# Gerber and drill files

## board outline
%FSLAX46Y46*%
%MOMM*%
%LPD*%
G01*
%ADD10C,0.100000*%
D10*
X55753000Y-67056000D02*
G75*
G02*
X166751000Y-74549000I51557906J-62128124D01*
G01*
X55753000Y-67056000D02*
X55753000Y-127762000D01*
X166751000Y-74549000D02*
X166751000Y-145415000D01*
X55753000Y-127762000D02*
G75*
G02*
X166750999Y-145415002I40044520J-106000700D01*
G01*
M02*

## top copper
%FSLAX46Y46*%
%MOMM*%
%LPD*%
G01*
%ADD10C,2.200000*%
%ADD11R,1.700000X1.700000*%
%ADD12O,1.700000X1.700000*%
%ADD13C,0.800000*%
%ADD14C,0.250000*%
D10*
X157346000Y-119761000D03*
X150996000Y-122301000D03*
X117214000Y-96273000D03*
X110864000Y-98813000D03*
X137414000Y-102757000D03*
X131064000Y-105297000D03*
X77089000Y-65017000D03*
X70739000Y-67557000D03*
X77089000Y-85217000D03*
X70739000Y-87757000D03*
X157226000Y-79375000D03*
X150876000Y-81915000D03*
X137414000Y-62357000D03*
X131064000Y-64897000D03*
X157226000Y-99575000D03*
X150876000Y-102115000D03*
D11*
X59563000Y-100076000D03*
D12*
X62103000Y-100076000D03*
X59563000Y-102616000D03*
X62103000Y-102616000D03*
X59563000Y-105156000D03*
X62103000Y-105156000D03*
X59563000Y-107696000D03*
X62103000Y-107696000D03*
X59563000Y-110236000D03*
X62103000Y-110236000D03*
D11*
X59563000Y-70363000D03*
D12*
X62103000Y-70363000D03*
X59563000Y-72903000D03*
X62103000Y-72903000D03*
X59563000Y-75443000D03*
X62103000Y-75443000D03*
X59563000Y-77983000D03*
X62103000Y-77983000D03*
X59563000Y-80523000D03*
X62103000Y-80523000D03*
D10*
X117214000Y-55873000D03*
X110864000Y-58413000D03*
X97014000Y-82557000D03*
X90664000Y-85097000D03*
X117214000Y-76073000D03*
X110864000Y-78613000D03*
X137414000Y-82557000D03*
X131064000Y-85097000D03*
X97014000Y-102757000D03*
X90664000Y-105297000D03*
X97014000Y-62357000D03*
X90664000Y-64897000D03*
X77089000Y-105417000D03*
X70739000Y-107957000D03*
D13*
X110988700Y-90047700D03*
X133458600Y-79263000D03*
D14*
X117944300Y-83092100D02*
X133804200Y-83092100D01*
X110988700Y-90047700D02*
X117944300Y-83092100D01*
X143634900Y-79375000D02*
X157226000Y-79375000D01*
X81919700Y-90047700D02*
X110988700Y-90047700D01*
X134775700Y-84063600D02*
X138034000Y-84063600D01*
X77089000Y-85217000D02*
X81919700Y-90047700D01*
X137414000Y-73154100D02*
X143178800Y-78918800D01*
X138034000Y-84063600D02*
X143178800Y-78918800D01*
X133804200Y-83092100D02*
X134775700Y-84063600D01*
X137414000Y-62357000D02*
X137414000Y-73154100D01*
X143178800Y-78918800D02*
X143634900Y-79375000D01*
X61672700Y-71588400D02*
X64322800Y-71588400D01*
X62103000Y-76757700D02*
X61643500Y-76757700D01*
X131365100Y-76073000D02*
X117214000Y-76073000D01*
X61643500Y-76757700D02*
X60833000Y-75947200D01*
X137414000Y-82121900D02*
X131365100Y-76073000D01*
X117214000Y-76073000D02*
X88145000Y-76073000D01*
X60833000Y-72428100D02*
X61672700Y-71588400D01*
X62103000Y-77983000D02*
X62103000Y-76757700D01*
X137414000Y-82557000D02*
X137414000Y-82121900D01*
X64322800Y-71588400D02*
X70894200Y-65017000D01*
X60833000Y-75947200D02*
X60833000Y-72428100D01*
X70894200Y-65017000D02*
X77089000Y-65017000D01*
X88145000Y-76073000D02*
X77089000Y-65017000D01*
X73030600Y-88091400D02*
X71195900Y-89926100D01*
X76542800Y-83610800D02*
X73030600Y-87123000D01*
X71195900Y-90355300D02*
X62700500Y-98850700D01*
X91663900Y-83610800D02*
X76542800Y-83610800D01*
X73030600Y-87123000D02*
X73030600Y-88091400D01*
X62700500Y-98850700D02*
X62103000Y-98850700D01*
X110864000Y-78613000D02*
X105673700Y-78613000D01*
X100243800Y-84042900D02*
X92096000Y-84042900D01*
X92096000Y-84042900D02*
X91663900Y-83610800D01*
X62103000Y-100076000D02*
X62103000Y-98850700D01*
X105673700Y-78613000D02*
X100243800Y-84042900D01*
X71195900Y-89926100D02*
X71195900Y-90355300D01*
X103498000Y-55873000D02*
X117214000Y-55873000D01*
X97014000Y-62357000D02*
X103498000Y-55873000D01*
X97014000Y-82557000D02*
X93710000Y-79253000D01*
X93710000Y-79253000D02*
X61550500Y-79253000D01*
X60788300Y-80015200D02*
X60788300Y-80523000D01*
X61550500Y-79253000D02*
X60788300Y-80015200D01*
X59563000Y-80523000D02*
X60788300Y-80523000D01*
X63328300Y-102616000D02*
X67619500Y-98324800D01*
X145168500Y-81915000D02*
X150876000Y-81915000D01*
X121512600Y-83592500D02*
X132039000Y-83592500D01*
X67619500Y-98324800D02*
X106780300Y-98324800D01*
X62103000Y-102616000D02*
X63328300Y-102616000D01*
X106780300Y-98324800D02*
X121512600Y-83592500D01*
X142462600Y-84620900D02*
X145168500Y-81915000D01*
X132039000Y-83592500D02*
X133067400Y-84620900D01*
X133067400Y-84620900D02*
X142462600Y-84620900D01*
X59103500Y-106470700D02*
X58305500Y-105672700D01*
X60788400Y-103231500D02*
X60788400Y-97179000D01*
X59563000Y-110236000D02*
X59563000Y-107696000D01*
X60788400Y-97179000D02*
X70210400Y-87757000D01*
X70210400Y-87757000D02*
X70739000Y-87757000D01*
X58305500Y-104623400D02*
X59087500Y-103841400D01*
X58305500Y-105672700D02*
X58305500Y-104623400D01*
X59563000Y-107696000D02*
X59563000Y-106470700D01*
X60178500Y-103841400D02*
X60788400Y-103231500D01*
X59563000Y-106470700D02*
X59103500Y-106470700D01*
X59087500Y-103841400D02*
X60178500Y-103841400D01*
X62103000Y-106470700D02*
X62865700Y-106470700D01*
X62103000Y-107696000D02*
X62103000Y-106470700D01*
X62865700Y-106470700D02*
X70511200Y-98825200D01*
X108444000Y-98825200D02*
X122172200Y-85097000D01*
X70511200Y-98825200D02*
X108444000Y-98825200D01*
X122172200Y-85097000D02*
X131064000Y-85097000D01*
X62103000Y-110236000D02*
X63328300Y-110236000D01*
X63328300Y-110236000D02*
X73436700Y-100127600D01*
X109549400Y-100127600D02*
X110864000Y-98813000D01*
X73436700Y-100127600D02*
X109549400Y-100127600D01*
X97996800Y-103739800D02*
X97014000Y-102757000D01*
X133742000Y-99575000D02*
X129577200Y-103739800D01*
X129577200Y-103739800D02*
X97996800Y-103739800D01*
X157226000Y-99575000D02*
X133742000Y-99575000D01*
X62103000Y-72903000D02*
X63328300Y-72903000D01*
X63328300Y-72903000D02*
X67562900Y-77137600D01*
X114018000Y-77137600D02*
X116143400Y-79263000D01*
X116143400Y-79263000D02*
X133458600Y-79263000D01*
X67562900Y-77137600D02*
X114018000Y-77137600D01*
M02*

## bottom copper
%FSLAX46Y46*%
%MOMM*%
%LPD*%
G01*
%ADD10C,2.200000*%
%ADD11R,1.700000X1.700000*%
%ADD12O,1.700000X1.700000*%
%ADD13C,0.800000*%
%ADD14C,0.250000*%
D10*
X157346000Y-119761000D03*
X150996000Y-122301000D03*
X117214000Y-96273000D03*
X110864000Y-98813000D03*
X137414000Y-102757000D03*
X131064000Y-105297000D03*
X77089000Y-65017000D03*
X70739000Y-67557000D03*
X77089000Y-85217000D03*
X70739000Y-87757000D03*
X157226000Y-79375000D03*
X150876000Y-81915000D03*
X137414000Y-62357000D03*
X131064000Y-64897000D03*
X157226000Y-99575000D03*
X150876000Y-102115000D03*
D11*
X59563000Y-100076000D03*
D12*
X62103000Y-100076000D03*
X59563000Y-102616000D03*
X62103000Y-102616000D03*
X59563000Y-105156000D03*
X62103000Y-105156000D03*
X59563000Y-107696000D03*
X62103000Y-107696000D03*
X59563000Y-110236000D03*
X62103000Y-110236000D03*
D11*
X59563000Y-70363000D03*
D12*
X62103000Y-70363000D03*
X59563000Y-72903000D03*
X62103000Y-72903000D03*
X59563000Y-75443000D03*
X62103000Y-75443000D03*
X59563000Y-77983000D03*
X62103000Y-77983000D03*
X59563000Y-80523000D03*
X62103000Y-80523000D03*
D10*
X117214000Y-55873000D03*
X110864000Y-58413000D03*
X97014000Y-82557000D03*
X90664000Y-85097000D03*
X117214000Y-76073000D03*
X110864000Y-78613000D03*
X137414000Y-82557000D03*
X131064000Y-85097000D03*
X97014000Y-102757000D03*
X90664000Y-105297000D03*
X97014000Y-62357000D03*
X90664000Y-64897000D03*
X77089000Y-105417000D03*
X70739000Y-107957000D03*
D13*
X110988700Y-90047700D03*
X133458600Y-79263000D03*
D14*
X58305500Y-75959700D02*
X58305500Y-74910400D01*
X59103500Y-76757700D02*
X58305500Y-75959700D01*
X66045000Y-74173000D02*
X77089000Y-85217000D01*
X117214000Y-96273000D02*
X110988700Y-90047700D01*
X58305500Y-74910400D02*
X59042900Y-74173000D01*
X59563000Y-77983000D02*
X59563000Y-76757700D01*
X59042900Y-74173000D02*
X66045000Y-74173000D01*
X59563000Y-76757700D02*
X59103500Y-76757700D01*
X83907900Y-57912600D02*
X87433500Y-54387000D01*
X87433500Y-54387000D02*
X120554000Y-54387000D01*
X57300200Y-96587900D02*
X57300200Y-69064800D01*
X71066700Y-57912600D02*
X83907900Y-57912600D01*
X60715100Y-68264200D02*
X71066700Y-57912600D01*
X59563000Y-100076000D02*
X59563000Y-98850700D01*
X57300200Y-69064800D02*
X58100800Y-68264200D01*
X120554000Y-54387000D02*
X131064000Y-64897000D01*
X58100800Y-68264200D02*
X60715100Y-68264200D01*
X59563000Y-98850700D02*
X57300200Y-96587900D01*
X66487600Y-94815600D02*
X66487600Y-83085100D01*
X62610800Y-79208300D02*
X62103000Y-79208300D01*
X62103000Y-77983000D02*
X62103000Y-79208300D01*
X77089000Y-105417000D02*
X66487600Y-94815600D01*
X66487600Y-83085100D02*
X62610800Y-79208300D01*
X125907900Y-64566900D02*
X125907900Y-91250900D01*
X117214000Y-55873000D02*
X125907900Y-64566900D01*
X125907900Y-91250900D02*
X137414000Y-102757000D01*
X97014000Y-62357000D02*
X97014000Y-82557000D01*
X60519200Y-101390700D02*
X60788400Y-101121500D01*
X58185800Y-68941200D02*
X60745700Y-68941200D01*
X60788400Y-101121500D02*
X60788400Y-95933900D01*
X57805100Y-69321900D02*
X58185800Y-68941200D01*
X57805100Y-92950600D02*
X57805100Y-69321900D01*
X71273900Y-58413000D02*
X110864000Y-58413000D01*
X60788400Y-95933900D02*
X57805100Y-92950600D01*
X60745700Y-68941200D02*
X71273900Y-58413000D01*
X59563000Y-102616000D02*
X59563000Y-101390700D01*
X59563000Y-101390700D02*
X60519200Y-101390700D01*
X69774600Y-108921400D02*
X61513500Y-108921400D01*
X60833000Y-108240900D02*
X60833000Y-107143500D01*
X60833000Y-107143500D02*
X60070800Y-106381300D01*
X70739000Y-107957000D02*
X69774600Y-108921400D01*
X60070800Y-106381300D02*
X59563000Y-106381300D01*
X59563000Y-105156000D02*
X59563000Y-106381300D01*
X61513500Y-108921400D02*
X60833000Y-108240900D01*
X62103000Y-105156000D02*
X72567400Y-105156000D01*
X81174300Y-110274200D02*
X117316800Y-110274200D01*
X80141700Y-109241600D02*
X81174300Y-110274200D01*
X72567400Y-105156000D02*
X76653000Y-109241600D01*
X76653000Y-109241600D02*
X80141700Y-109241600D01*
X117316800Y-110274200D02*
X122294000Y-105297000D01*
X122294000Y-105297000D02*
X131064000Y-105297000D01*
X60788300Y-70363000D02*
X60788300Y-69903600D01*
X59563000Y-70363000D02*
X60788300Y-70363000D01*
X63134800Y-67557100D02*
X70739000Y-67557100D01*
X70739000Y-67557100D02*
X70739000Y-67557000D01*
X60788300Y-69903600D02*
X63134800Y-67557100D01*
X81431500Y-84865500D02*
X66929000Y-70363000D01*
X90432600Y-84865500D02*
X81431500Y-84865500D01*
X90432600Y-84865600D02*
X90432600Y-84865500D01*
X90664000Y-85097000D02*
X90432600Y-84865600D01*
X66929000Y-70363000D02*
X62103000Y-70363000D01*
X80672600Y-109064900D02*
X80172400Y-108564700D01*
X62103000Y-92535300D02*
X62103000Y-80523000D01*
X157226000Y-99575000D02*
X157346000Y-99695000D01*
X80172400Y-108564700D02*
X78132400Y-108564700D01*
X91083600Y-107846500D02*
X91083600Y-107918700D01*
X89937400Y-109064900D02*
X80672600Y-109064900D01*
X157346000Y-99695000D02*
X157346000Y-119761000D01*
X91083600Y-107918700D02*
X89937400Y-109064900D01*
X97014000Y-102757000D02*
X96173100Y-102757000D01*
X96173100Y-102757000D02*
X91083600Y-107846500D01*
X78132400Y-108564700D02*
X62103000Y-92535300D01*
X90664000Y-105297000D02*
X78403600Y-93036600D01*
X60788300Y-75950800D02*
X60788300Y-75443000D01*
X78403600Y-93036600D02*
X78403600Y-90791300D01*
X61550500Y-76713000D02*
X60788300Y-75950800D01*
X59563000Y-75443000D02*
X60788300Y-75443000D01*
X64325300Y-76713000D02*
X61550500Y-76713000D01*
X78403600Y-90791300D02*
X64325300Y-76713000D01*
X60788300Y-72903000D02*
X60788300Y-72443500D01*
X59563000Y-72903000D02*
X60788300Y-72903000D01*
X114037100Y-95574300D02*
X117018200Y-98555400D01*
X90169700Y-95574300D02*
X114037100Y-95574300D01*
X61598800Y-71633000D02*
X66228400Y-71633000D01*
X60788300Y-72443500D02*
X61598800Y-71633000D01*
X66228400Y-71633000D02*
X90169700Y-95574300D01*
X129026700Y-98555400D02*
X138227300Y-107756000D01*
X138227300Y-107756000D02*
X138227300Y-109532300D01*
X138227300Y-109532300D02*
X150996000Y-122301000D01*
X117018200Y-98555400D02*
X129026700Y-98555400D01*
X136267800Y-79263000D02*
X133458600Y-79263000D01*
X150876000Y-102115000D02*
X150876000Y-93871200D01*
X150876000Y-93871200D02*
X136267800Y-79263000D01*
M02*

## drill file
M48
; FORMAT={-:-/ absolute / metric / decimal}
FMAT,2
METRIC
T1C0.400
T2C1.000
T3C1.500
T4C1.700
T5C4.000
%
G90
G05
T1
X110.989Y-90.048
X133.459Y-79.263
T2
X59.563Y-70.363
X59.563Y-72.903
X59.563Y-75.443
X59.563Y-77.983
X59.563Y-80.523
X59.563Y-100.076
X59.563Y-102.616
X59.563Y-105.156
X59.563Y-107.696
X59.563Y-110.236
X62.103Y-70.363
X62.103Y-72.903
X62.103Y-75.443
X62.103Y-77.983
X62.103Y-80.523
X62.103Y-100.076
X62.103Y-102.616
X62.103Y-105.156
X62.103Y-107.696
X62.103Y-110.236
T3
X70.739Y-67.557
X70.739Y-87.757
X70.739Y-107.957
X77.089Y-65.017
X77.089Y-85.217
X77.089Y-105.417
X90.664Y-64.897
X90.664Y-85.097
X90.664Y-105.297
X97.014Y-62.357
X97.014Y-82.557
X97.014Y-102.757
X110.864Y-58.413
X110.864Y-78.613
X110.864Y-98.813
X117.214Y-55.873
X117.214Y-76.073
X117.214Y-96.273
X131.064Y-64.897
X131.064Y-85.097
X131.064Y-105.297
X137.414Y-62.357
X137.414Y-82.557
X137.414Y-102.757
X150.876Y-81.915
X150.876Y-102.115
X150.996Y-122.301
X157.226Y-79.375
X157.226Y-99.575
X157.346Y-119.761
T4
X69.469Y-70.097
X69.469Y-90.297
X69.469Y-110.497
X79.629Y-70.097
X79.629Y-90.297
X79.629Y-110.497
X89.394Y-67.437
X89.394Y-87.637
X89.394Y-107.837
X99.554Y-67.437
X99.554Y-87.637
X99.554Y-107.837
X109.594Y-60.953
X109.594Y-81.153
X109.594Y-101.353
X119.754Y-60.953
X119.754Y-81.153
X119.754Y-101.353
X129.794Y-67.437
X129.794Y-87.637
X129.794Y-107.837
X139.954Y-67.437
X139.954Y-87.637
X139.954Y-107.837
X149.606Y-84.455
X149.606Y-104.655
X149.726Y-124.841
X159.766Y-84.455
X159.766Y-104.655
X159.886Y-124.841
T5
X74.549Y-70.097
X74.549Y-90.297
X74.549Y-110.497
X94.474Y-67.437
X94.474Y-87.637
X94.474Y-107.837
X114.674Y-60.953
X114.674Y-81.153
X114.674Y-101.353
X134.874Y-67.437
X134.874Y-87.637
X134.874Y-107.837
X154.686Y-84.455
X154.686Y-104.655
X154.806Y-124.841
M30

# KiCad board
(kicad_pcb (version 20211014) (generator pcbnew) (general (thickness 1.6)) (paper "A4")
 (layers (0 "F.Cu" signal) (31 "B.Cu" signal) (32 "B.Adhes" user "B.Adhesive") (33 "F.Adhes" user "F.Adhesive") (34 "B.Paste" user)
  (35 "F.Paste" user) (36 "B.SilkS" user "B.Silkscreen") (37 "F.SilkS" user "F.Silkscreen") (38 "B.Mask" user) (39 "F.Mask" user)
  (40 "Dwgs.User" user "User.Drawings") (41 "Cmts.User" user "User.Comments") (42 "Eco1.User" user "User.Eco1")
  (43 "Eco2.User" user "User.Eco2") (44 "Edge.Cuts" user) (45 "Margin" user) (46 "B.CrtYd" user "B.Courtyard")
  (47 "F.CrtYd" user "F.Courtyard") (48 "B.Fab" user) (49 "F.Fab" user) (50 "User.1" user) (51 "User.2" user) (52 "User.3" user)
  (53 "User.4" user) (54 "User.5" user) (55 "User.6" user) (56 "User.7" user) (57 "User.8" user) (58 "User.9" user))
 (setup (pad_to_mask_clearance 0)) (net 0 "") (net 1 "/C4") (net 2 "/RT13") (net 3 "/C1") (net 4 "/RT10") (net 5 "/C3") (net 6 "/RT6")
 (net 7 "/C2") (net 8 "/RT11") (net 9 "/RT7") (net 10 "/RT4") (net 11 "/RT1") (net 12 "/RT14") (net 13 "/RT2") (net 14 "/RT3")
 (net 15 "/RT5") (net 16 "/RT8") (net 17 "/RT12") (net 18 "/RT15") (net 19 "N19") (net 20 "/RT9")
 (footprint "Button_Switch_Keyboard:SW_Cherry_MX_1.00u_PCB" (layer "F.Cu") (at 157.346 119.761)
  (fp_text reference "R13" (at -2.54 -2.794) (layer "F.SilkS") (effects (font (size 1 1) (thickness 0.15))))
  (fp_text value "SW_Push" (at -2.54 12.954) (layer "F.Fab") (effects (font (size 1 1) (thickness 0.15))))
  (pad "" np_thru_hole circle (at 2.54 5.08) (size 1.7 1.7) (drill 1.7) (layers *.Cu *.Mask))
  (pad "" np_thru_hole circle (at -2.54 5.08) (size 4 4) (drill 4) (layers *.Cu *.Mask))
  (pad "" np_thru_hole circle (at -7.62 5.08) (size 1.7 1.7) (drill 1.7) (layers *.Cu *.Mask))
  (pad "1" thru_hole circle (at 0 0) (size 2.2 2.2) (drill 1.5) (layers *.Cu *.Mask) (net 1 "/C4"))
  (pad "2" thru_hole circle (at -6.35 2.54) (size 2.2 2.2) (drill 1.5) (layers *.Cu *.Mask) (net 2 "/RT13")))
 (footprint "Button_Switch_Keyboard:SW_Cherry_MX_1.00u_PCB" (layer "F.Cu") (at 117.214 96.273)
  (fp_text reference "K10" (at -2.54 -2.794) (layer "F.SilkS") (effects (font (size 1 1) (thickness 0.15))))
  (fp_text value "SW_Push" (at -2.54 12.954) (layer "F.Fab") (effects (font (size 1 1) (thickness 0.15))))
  (pad "" np_thru_hole circle (at 2.54 5.08) (size 1.7 1.7) (drill 1.7) (layers *.Cu *.Mask))
  (pad "" np_thru_hole circle (at -7.62 5.08) (size 1.7 1.7) (drill 1.7) (layers *.Cu *.Mask))
  (pad "" np_thru_hole circle (at -2.54 5.08) (size 4 4) (drill 4) (layers *.Cu *.Mask))
  (pad "1" thru_hole circle (at 0 0) (size 2.2 2.2) (drill 1.5) (layers *.Cu *.Mask) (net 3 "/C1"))
  (pad "2" thru_hole circle (at -6.35 2.54) (size 2.2 2.2) (drill 1.5) (layers *.Cu *.Mask) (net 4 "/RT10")))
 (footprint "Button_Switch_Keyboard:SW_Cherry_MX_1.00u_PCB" (layer "F.Cu") (at 137.414 102.757)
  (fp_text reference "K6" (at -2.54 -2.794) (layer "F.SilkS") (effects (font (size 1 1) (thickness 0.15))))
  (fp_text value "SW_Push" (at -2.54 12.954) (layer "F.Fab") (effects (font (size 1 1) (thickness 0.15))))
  (pad "" np_thru_hole circle (at -7.62 5.08) (size 1.7 1.7) (drill 1.7) (layers *.Cu *.Mask))
  (pad "" np_thru_hole circle (at 2.54 5.08) (size 1.7 1.7) (drill 1.7) (layers *.Cu *.Mask))
  (pad "" np_thru_hole circle (at -2.54 5.08) (size 4 4) (drill 4) (layers *.Cu *.Mask))
  (pad "1" thru_hole circle (at 0 0) (size 2.2 2.2) (drill 1.5) (layers *.Cu *.Mask) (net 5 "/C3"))
  (pad "2" thru_hole circle (at -6.35 2.54) (size 2.2 2.2) (drill 1.5) (layers *.Cu *.Mask) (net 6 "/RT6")))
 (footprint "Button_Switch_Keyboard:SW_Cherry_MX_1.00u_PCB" (layer "F.Cu") (at 77.089 65.017)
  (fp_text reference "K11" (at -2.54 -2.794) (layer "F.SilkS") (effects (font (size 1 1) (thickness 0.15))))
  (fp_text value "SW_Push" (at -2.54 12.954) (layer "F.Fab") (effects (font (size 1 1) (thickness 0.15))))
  (pad "" np_thru_hole circle (at 2.54 5.08) (size 1.7 1.7) (drill 1.7) (layers *.Cu *.Mask))
  (pad "" np_thru_hole circle (at -7.62 5.08) (size 1.7 1.7) (drill 1.7) (layers *.Cu *.Mask))
  (pad "" np_thru_hole circle (at -2.54 5.08) (size 4 4) (drill 4) (layers *.Cu *.Mask))
  (pad "1" thru_hole circle (at 0 0) (size 2.2 2.2) (drill 1.5) (layers *.Cu *.Mask) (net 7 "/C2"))
  (pad "2" thru_hole circle (at -6.35 2.54) (size 2.2 2.2) (drill 1.5) (layers *.Cu *.Mask) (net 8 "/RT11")))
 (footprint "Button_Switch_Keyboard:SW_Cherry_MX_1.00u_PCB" (layer "F.Cu") (at 77.089 85.217)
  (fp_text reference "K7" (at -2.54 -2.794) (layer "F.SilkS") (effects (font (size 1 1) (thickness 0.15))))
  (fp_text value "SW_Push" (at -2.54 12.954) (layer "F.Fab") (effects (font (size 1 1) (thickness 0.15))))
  (pad "" np_thru_hole circle (at -7.62 5.08) (size 1.7 1.7) (drill 1.7) (layers *.Cu *.Mask))
  (pad "" np_thru_hole circle (at -2.54 5.08) (size 4 4) (drill 4) (layers *.Cu *.Mask))
  (pad "" np_thru_hole circle (at 2.54 5.08) (size 1.7 1.7) (drill 1.7) (layers *.Cu *.Mask))
  (pad "1" thru_hole circle (at 0 0) (size 2.2 2.2) (drill 1.5) (layers *.Cu *.Mask) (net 3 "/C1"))
  (pad "2" thru_hole circle (at -6.35 2.54) (size 2.2 2.2) (drill 1.5) (layers *.Cu *.Mask) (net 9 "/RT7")))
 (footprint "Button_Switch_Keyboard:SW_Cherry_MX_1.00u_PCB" (layer "F.Cu") (at 157.226 79.375)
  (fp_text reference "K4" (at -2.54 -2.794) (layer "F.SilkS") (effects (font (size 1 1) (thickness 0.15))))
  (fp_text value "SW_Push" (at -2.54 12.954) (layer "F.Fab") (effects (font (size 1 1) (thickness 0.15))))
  (pad "" np_thru_hole circle (at 2.54 5.08) (size 1.7 1.7) (drill 1.7) (layers *.Cu *.Mask))
  (pad "" np_thru_hole circle (at -7.62 5.08) (size 1.7 1.7) (drill 1.7) (layers *.Cu *.Mask))
  (pad "" np_thru_hole circle (at -2.54 5.08) (size 4 4) (drill 4) (layers *.Cu *.Mask))
  (pad "1" thru_hole circle (at 0 0) (size 2.2 2.2) (drill 1.5) (layers *.Cu *.Mask) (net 3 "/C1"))
  (pad "2" thru_hole circle (at -6.35 2.54) (size 2.2 2.2) (drill 1.5) (layers *.Cu *.Mask) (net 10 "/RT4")))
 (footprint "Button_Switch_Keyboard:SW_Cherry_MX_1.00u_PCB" (layer "F.Cu") (at 137.414 62.357)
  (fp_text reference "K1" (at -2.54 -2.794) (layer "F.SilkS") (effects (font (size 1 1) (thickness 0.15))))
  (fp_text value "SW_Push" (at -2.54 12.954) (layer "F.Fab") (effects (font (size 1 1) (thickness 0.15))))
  (pad "" np_thru_hole circle (at -2.54 5.08) (size 4 4) (drill 4) (layers *.Cu *.Mask))
  (pad "" np_thru_hole circle (at -7.62 5.08) (size 1.7 1.7) (drill 1.7) (layers *.Cu *.Mask))
  (pad "" np_thru_hole circle (at 2.54 5.08) (size 1.7 1.7) (drill 1.7) (layers *.Cu *.Mask))
  (pad "1" thru_hole circle (at 0 0) (size 2.2 2.2) (drill 1.5) (layers *.Cu *.Mask) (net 3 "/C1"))
  (pad "2" thru_hole circle (at -6.35 2.54) (size 2.2 2.2) (drill 1.5) (layers *.Cu *.Mask) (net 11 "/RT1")))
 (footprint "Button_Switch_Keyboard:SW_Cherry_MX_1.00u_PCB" (layer "F.Cu") (at 157.226 99.575)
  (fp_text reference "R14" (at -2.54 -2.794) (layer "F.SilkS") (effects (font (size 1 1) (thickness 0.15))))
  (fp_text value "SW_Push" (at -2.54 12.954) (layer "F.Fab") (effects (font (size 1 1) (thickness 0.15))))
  (pad "" np_thru_hole circle (at -7.62 5.08) (size 1.7 1.7) (drill 1.7) (layers *.Cu *.Mask))
  (pad "" np_thru_hole circle (at -2.54 5.08) (size 4 4) (drill 4) (layers *.Cu *.Mask))
  (pad "" np_thru_hole circle (at 2.54 5.08) (size 1.7 1.7) (drill 1.7) (layers *.Cu *.Mask))
  (pad "1" thru_hole circle (at 0 0) (size 2.2 2.2) (drill 1.5) (layers *.Cu *.Mask) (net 1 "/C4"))
  (pad "2" thru_hole circle (at -6.35 2.54) (size 2.2 2.2) (drill 1.5) (layers *.Cu *.Mask) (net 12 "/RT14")))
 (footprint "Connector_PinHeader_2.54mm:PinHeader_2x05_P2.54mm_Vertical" (layer "F.Cu") (at 59.563 100.076)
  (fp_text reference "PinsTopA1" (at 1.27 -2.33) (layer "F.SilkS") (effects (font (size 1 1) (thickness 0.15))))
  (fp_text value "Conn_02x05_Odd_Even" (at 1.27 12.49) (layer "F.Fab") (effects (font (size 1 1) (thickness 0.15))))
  (pad "1" thru_hole rect (at 0 0) (size 1.7 1.7) (drill 1) (layers *.Cu *.Mask) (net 11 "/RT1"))
  (pad "2" thru_hole oval (at 2.54 0) (size 1.7 1.7) (drill 1) (layers *.Cu *.Mask) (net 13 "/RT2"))
  (pad "3" thru_hole oval (at 0 2.54) (size 1.7 1.7) (drill 1) (layers *.Cu *.Mask) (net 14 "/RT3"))
  (pad "4" thru_hole oval (at 2.54 2.54) (size 1.7 1.7) (drill 1) (layers *.Cu *.Mask) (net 10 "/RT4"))
  (pad "5" thru_hole oval (at 0 5.08) (size 1.7 1.7) (drill 1) (layers *.Cu *.Mask) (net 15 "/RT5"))
  (pad "6" thru_hole oval (at 2.54 5.08) (size 1.7 1.7) (drill 1) (layers *.Cu *.Mask) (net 6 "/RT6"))
  (pad "7" thru_hole oval (at 0 7.62) (size 1.7 1.7) (drill 1) (layers *.Cu *.Mask) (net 9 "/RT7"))
  (pad "8" thru_hole oval (at 2.54 7.62) (size 1.7 1.7) (drill 1) (layers *.Cu *.Mask) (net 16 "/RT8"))
  (pad "9" thru_hole oval (at 0 10.16) (size 1.7 1.7) (drill 1) (layers *.Cu *.Mask) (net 9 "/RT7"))
  (pad "10" thru_hole oval (at 2.54 10.16) (size 1.7 1.7) (drill 1) (layers *.Cu *.Mask) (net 4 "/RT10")))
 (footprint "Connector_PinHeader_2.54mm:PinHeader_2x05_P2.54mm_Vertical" (layer "F.Cu") (at 59.563 70.363)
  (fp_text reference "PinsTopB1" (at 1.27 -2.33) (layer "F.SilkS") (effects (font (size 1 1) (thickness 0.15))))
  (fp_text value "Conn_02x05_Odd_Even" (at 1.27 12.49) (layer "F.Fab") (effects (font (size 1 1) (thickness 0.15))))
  (pad "1" thru_hole rect (at 0 0) (size 1.7 1.7) (drill 1) (layers *.Cu *.Mask) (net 8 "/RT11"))
  (pad "2" thru_hole oval (at 2.54 0) (size 1.7 1.7) (drill 1) (layers *.Cu *.Mask) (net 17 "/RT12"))
  (pad "3" thru_hole oval (at 0 2.54) (size 1.7 1.7) (drill 1) (layers *.Cu *.Mask) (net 2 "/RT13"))
  (pad "4" thru_hole oval (at 2.54 2.54) (size 1.7 1.7) (drill 1) (layers *.Cu *.Mask) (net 12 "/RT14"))
  (pad "5" thru_hole oval (at 0 5.08) (size 1.7 1.7) (drill 1) (layers *.Cu *.Mask) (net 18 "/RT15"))
  (pad "6" thru_hole oval (at 2.54 5.08) (size 1.7 1.7) (drill 1) (layers *.Cu *.Mask) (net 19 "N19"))
  (pad "7" thru_hole oval (at 0 7.62) (size 1.7 1.7) (drill 1) (layers *.Cu *.Mask) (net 3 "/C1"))
  (pad "8" thru_hole oval (at 2.54 7.62) (size 1.7 1.7) (drill 1) (layers *.Cu *.Mask) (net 7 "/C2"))
  (pad "9" thru_hole oval (at 0 10.16) (size 1.7 1.7) (drill 1) (layers *.Cu *.Mask) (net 5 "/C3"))
  (pad "10" thru_hole oval (at 2.54 10.16) (size 1.7 1.7) (drill 1) (layers *.Cu *.Mask) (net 1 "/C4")))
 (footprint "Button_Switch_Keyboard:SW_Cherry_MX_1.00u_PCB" (layer "F.Cu") (at 117.214 55.873)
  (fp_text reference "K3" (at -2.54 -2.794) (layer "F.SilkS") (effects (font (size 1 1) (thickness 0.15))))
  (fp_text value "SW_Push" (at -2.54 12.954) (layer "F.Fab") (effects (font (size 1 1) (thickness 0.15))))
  (pad "" np_thru_hole circle (at 2.54 5.08) (size 1.7 1.7) (drill 1.7) (layers *.Cu *.Mask))
  (pad "" np_thru_hole circle (at -7.62 5.08) (size 1.7 1.7) (drill 1.7) (layers *.Cu *.Mask))
  (pad "" np_thru_hole circle (at -2.54 5.08) (size 4 4) (drill 4) (layers *.Cu *.Mask))
  (pad "1" thru_hole circle (at 0 0) (size 2.2 2.2) (drill 1.5) (layers *.Cu *.Mask) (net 5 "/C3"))
  (pad "2" thru_hole circle (at -6.35 2.54) (size 2.2 2.2) (drill 1.5) (layers *.Cu *.Mask) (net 14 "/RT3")))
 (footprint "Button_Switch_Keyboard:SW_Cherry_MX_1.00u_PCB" (layer "F.Cu") (at 97.014 82.557)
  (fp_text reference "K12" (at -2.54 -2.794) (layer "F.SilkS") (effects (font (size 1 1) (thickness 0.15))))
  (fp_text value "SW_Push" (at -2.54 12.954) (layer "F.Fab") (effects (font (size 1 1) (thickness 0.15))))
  (pad "" np_thru_hole circle (at 2.54 5.08) (size 1.7 1.7) (drill 1.7) (layers *.Cu *.Mask))
  (pad "" np_thru_hole circle (at -7.62 5.08) (size 1.7 1.7) (drill 1.7) (layers *.Cu *.Mask))
  (pad "" np_thru_hole circle (at -2.54 5.08) (size 4 4) (drill 4) (layers *.Cu *.Mask))
  (pad "1" thru_hole circle (at 0 0) (size 2.2 2.2) (drill 1.5) (layers *.Cu *.Mask) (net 5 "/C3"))
  (pad "2" thru_hole circle (at -6.35 2.54) (size 2.2 2.2) (drill 1.5) (layers *.Cu *.Mask) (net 17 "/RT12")))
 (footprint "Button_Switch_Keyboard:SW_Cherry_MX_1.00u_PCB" (layer "F.Cu") (at 117.214 76.073)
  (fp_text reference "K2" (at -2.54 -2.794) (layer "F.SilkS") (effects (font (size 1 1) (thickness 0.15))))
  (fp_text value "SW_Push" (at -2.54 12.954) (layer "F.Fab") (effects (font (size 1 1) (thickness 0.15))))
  (pad "" np_thru_hole circle (at -7.62 5.08) (size 1.7 1.7) (drill 1.7) (layers *.Cu *.Mask))
  (pad "" np_thru_hole circle (at -2.54 5.08) (size 4 4) (drill 4) (layers *.Cu *.Mask))
  (pad "" np_thru_hole circle (at 2.54 5.08) (size 1.7 1.7) (drill 1.7) (layers *.Cu *.Mask))
  (pad "1" thru_hole circle (at 0 0) (size 2.2 2.2) (drill 1.5) (layers *.Cu *.Mask) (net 7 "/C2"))
  (pad "2" thru_hole circle (at -6.35 2.54) (size 2.2 2.2) (drill 1.5) (layers *.Cu *.Mask) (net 13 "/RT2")))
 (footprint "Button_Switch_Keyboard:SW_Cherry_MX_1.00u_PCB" (layer "F.Cu") (at 137.414 82.557)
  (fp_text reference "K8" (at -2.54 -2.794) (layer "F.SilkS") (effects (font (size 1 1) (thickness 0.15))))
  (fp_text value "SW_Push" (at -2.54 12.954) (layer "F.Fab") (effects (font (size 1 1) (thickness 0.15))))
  (pad "" np_thru_hole circle (at -2.54 5.08) (size 4 4) (drill 4) (layers *.Cu *.Mask))
  (pad "" np_thru_hole circle (at 2.54 5.08) (size 1.7 1.7) (drill 1.7) (layers *.Cu *.Mask))
  (pad "" np_thru_hole circle (at -7.62 5.08) (size 1.7 1.7) (drill 1.7) (layers *.Cu *.Mask))
  (pad "1" thru_hole circle (at 0 0) (size 2.2 2.2) (drill 1.5) (layers *.Cu *.Mask) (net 7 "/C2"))
  (pad "2" thru_hole circle (at -6.35 2.54) (size 2.2 2.2) (drill 1.5) (layers *.Cu *.Mask) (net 16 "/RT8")))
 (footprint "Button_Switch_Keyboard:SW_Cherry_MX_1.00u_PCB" (layer "F.Cu") (at 97.014 102.757)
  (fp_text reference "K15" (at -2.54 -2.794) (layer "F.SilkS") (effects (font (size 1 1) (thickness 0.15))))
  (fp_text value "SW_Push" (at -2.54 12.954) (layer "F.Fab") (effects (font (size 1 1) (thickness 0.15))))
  (pad "" np_thru_hole circle (at 2.54 5.08) (size 1.7 1.7) (drill 1.7) (layers *.Cu *.Mask))
  (pad "" np_thru_hole circle (at -2.54 5.08) (size 4 4) (drill 4) (layers *.Cu *.Mask))
  (pad "" np_thru_hole circle (at -7.62 5.08) (size 1.7 1.7) (drill 1.7) (layers *.Cu *.Mask))
  (pad "1" thru_hole circle (at 0 0) (size 2.2 2.2) (drill 1.5) (layers *.Cu *.Mask) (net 1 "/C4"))
  (pad "2" thru_hole circle (at -6.35 2.54) (size 2.2 2.2) (drill 1.5) (layers *.Cu *.Mask) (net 18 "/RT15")))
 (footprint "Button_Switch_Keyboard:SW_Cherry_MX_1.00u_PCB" (layer "F.Cu") (at 97.014 62.357)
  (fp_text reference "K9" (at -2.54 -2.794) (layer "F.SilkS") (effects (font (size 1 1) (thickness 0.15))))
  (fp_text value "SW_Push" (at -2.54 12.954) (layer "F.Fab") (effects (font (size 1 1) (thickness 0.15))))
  (pad "" np_thru_hole circle (at -7.62 5.08) (size 1.7 1.7) (drill 1.7) (layers *.Cu *.Mask))
  (pad "" np_thru_hole circle (at -2.54 5.08) (size 4 4) (drill 4) (layers *.Cu *.Mask))
  (pad "" np_thru_hole circle (at 2.54 5.08) (size 1.7 1.7) (drill 1.7) (layers *.Cu *.Mask))
  (pad "1" thru_hole circle (at 0 0) (size 2.2 2.2) (drill 1.5) (layers *.Cu *.Mask) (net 5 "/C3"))
  (pad "2" thru_hole circle (at -6.35 2.54) (size 2.2 2.2) (drill 1.5) (layers *.Cu *.Mask) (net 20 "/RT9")))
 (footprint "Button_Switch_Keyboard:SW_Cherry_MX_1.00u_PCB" (layer "F.Cu") (at 77.089 105.417)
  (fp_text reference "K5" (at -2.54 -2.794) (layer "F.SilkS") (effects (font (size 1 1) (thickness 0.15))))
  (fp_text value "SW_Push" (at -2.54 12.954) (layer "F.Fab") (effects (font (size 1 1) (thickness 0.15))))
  (pad "" np_thru_hole circle (at -2.54 5.08) (size 4 4) (drill 4) (layers *.Cu *.Mask))
  (pad "" np_thru_hole circle (at 2.54 5.08) (size 1.7 1.7) (drill 1.7) (layers *.Cu *.Mask))
  (pad "" np_thru_hole circle (at -7.62 5.08) (size 1.7 1.7) (drill 1.7) (layers *.Cu *.Mask))
  (pad "1" thru_hole circle (at 0 0) (size 2.2 2.2) (drill 1.5) (layers *.Cu *.Mask) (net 7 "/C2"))
  (pad "2" thru_hole circle (at -6.35 2.54) (size 2.2 2.2) (drill 1.5) (layers *.Cu *.Mask) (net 15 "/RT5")))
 (gr_arc (start 55.753 67.056) (mid 112.748597 48.632569) (end 166.751 74.549) (layer "Edge.Cuts") (width 0.1))
 (gr_line (start 55.753 67.056) (end 55.753 127.762) (layer "Edge.Cuts") (width 0.1))
 (gr_line (start 166.751 74.549) (end 166.751 145.415) (layer "Edge.Cuts") (width 0.1))
 (gr_arc (start 55.753 127.762) (mid 113.594937 121.85665) (end 166.751 145.415) (layer "Edge.Cuts") (width 0.1))
 (segment (start 117.9443 83.0921) (end 133.8042 83.0921) (width 0.25) (layer "F.Cu") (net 3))
 (segment (start 110.9887 90.0477) (end 117.9443 83.0921) (width 0.25) (layer "F.Cu") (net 3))
 (segment (start 143.6349 79.375) (end 157.226 79.375) (width 0.25) (layer "F.Cu") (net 3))
 (segment (start 81.9197 90.0477) (end 110.9887 90.0477) (width 0.25) (layer "F.Cu") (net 3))
 (segment (start 134.7757 84.0636) (end 138.034 84.0636) (width 0.25) (layer "F.Cu") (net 3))
 (segment (start 77.089 85.217) (end 81.9197 90.0477) (width 0.25) (layer "F.Cu") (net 3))
 (segment (start 137.414 73.1541) (end 143.1788 78.9188) (width 0.25) (layer "F.Cu") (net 3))
 (segment (start 138.034 84.0636) (end 143.1788 78.9188) (width 0.25) (layer "F.Cu") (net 3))
 (segment (start 133.8042 83.0921) (end 134.7757 84.0636) (width 0.25) (layer "F.Cu") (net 3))
 (segment (start 137.414 62.357) (end 137.414 73.1541) (width 0.25) (layer "F.Cu") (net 3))
 (segment (start 143.1788 78.9188) (end 143.6349 79.375) (width 0.25) (layer "F.Cu") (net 3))
 (via (at 110.9887 90.0477) (size 0.8) (drill 0.4) (layers "F.Cu" "B.Cu") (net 3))
 (segment (start 58.3055 75.9597) (end 58.3055 74.9104) (width 0.25) (layer "B.Cu") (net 3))
 (segment (start 59.1035 76.7577) (end 58.3055 75.9597) (width 0.25) (layer "B.Cu") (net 3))
 (segment (start 66.045 74.173) (end 77.089 85.217) (width 0.25) (layer "B.Cu") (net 3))
 (segment (start 117.214 96.273) (end 110.9887 90.0477) (width 0.25) (layer "B.Cu") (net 3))
 (segment (start 58.3055 74.9104) (end 59.0429 74.173) (width 0.25) (layer "B.Cu") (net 3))
 (segment (start 59.563 77.983) (end 59.563 76.7577) (width 0.25) (layer "B.Cu") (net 3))
 (segment (start 59.0429 74.173) (end 66.045 74.173) (width 0.25) (layer "B.Cu") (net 3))
 (segment (start 59.563 76.7577) (end 59.1035 76.7577) (width 0.25) (layer "B.Cu") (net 3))
 (segment (start 83.9079 57.9126) (end 87.4335 54.387) (width 0.25) (layer "B.Cu") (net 11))
 (segment (start 87.4335 54.387) (end 120.554 54.387) (width 0.25) (layer "B.Cu") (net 11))
 (segment (start 57.3002 96.5879) (end 57.3002 69.0648) (width 0.25) (layer "B.Cu") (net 11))
 (segment (start 71.0667 57.9126) (end 83.9079 57.9126) (width 0.25) (layer "B.Cu") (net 11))
 (segment (start 60.7151 68.2642) (end 71.0667 57.9126) (width 0.25) (layer "B.Cu") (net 11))
 (segment (start 59.563 100.076) (end 59.563 98.8507) (width 0.25) (layer "B.Cu") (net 11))
 (segment (start 57.3002 69.0648) (end 58.1008 68.2642) (width 0.25) (layer "B.Cu") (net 11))
 (segment (start 120.554 54.387) (end 131.064 64.897) (width 0.25) (layer "B.Cu") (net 11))
 (segment (start 58.1008 68.2642) (end 60.7151 68.2642) (width 0.25) (layer "B.Cu") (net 11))
 (segment (start 59.563 98.8507) (end 57.3002 96.5879) (width 0.25) (layer "B.Cu") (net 11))
 (segment (start 61.6727 71.5884) (end 64.3228 71.5884) (width 0.25) (layer "F.Cu") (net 7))
 (segment (start 62.103 76.7577) (end 61.6435 76.7577) (width 0.25) (layer "F.Cu") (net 7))
 (segment (start 131.3651 76.073) (end 117.214 76.073) (width 0.25) (layer "F.Cu") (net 7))
 (segment (start 61.6435 76.7577) (end 60.833 75.9472) (width 0.25) (layer "F.Cu") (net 7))
 (segment (start 137.414 82.1219) (end 131.3651 76.073) (width 0.25) (layer "F.Cu") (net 7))
 (segment (start 117.214 76.073) (end 88.145 76.073) (width 0.25) (layer "F.Cu") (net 7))
 (segment (start 60.833 72.4281) (end 61.6727 71.5884) (width 0.25) (layer "F.Cu") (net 7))
 (segment (start 62.103 77.983) (end 62.103 76.7577) (width 0.25) (layer "F.Cu") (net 7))
 (segment (start 137.414 82.557) (end 137.414 82.1219) (width 0.25) (layer "F.Cu") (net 7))
 (segment (start 64.3228 71.5884) (end 70.8942 65.017) (width 0.25) (layer "F.Cu") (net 7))
 (segment (start 60.833 75.9472) (end 60.833 72.4281) (width 0.25) (layer "F.Cu") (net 7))
 (segment (start 70.8942 65.017) (end 77.089 65.017) (width 0.25) (layer "F.Cu") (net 7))
 (segment (start 88.145 76.073) (end 77.089 65.017) (width 0.25) (layer "F.Cu") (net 7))
 (segment (start 66.4876 94.8156) (end 66.4876 83.0851) (width 0.25) (layer "B.Cu") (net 7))
 (segment (start 62.6108 79.2083) (end 62.103 79.2083) (width 0.25) (layer "B.Cu") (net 7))
 (segment (start 62.103 77.983) (end 62.103 79.2083) (width 0.25) (layer "B.Cu") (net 7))
 (segment (start 77.089 105.417) (end 66.4876 94.8156) (width 0.25) (layer "B.Cu") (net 7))
 (segment (start 66.4876 83.0851) (end 62.6108 79.2083) (width 0.25) (layer "B.Cu") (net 7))
 (segment (start 73.0306 88.0914) (end 71.1959 89.9261) (width 0.25) (layer "F.Cu") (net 13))
 (segment (start 76.5428 83.6108) (end 73.0306 87.123) (width 0.25) (layer "F.Cu") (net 13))
 (segment (start 71.1959 90.3553) (end 62.7005 98.8507) (width 0.25) (layer "F.Cu") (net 13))
 (segment (start 91.6639 83.6108) (end 76.5428 83.6108) (width 0.25) (layer "F.Cu") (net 13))
 (segment (start 73.0306 87.123) (end 73.0306 88.0914) (width 0.25) (layer "F.Cu") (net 13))
 (segment (start 62.7005 98.8507) (end 62.103 98.8507) (width 0.25) (layer "F.Cu") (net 13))
 (segment (start 110.864 78.613) (end 105.6737 78.613) (width 0.25) (layer "F.Cu") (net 13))
 (segment (start 100.2438 84.0429) (end 92.096 84.0429) (width 0.25) (layer "F.Cu") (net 13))
 (segment (start 92.096 84.0429) (end 91.6639 83.6108) (width 0.25) (layer "F.Cu") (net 13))
 (segment (start 62.103 100.076) (end 62.103 98.8507) (width 0.25) (layer "F.Cu") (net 13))
 (segment (start 105.6737 78.613) (end 100.2438 84.0429) (width 0.25) (layer "F.Cu") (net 13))
 (segment (start 71.1959 89.9261) (end 71.1959 90.3553) (width 0.25) (layer "F.Cu") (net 13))
 (segment (start 103.498 55.873) (end 117.214 55.873) (width 0.25) (layer "F.Cu") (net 5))
 (segment (start 97.014 62.357) (end 103.498 55.873) (width 0.25) (layer "F.Cu") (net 5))
 (segment (start 97.014 82.557) (end 93.71 79.253) (width 0.25) (layer "F.Cu") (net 5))
 (segment (start 93.71 79.253) (end 61.5505 79.253) (width 0.25) (layer "F.Cu") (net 5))
 (segment (start 60.7883 80.0152) (end 60.7883 80.523) (width 0.25) (layer "F.Cu") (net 5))
 (segment (start 61.5505 79.253) (end 60.7883 80.0152) (width 0.25) (layer "F.Cu") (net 5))
 (segment (start 59.563 80.523) (end 60.7883 80.523) (width 0.25) (layer "F.Cu") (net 5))
 (segment (start 125.9079 64.5669) (end 125.9079 91.2509) (width 0.25) (layer "B.Cu") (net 5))
 (segment (start 117.214 55.873) (end 125.9079 64.5669) (width 0.25) (layer "B.Cu") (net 5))
 (segment (start 125.9079 91.2509) (end 137.414 102.757) (width 0.25) (layer "B.Cu") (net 5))
 (segment (start 97.014 62.357) (end 97.014 82.557) (width 0.25) (layer "B.Cu") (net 5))
 (segment (start 60.5192 101.3907) (end 60.7884 101.1215) (width 0.25) (layer "B.Cu") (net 14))
 (segment (start 58.1858 68.9412) (end 60.7457 68.9412) (width 0.25) (layer "B.Cu") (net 14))
 (segment (start 60.7884 101.1215) (end 60.7884 95.9339) (width 0.25) (layer "B.Cu") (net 14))
 (segment (start 57.8051 69.3219) (end 58.1858 68.9412) (width 0.25) (layer "B.Cu") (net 14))
 (segment (start 57.8051 92.9506) (end 57.8051 69.3219) (width 0.25) (layer "B.Cu") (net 14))
 (segment (start 71.2739 58.413) (end 110.864 58.413) (width 0.25) (layer "B.Cu") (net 14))
 (segment (start 60.7884 95.9339) (end 57.8051 92.9506) (width 0.25) (layer "B.Cu") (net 14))
 (segment (start 60.7457 68.9412) (end 71.2739 58.413) (width 0.25) (layer "B.Cu") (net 14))
 (segment (start 59.563 102.616) (end 59.563 101.3907) (width 0.25) (layer "B.Cu") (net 14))
 (segment (start 59.563 101.3907) (end 60.5192 101.3907) (width 0.25) (layer "B.Cu") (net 14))
 (segment (start 63.3283 102.616) (end 67.6195 98.3248) (width 0.25) (layer "F.Cu") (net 10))
 (segment (start 145.1685 81.915) (end 150.876 81.915) (width 0.25) (layer "F.Cu") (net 10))
 (segment (start 121.5126 83.5925) (end 132.039 83.5925) (width 0.25) (layer "F.Cu") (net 10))
 (segment (start 67.6195 98.3248) (end 106.7803 98.3248) (width 0.25) (layer "F.Cu") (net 10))
 (segment (start 62.103 102.616) (end 63.3283 102.616) (width 0.25) (layer "F.Cu") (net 10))
 (segment (start 106.7803 98.3248) (end 121.5126 83.5925) (width 0.25) (layer "F.Cu") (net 10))
 (segment (start 142.4626 84.6209) (end 145.1685 81.915) (width 0.25) (layer "F.Cu") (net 10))
 (segment (start 132.039 83.5925) (end 133.0674 84.6209) (width 0.25) (layer "F.Cu") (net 10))
 (segment (start 133.0674 84.6209) (end 142.4626 84.6209) (width 0.25) (layer "F.Cu") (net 10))
 (segment (start 69.7746 108.9214) (end 61.5135 108.9214) (width 0.25) (layer "B.Cu") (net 15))
 (segment (start 60.833 108.2409) (end 60.833 107.1435) (width 0.25) (layer "B.Cu") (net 15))
 (segment (start 60.833 107.1435) (end 60.0708 106.3813) (width 0.25) (layer "B.Cu") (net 15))
 (segment (start 70.739 107.957) (end 69.7746 108.9214) (width 0.25) (layer "B.Cu") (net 15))
 (segment (start 60.0708 106.3813) (end 59.563 106.3813) (width 0.25) (layer "B.Cu") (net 15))
 (segment (start 59.563 105.156) (end 59.563 106.3813) (width 0.25) (layer "B.Cu") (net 15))
 (segment (start 61.5135 108.9214) (end 60.833 108.2409) (width 0.25) (layer "B.Cu") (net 15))
 (segment (start 62.103 105.156) (end 72.5674 105.156) (width 0.25) (layer "B.Cu") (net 6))
 (segment (start 81.1743 110.2742) (end 117.3168 110.2742) (width 0.25) (layer "B.Cu") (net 6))
 (segment (start 80.1417 109.2416) (end 81.1743 110.2742) (width 0.25) (layer "B.Cu") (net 6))
 (segment (start 72.5674 105.156) (end 76.653 109.2416) (width 0.25) (layer "B.Cu") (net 6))
 (segment (start 76.653 109.2416) (end 80.1417 109.2416) (width 0.25) (layer "B.Cu") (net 6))
 (segment (start 117.3168 110.2742) (end 122.294 105.297) (width 0.25) (layer "B.Cu") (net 6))
 (segment (start 122.294 105.297) (end 131.064 105.297) (width 0.25) (layer "B.Cu") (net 6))
 (segment (start 59.1035 106.4707) (end 58.3055 105.6727) (width 0.25) (layer "F.Cu") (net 9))
 (segment (start 60.7884 103.2315) (end 60.7884 97.179) (width 0.25) (layer "F.Cu") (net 9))
 (segment (start 59.563 110.236) (end 59.563 107.696) (width 0.25) (layer "F.Cu") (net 9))
 (segment (start 60.7884 97.179) (end 70.2104 87.757) (width 0.25) (layer "F.Cu") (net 9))
 (segment (start 70.2104 87.757) (end 70.739 87.757) (width 0.25) (layer "F.Cu") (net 9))
 (segment (start 58.3055 104.6234) (end 59.0875 103.8414) (width 0.25) (layer "F.Cu") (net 9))
 (segment (start 58.3055 105.6727) (end 58.3055 104.6234) (width 0.25) (layer "F.Cu") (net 9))
 (segment (start 59.563 107.696) (end 59.563 106.4707) (width 0.25) (layer "F.Cu") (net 9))
 (segment (start 60.1785 103.8414) (end 60.7884 103.2315) (width 0.25) (layer "F.Cu") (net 9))
 (segment (start 59.563 106.4707) (end 59.1035 106.4707) (width 0.25) (layer "F.Cu") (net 9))
 (segment (start 59.0875 103.8414) (end 60.1785 103.8414) (width 0.25) (layer "F.Cu") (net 9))
 (segment (start 62.103 106.4707) (end 62.8657 106.4707) (width 0.25) (layer "F.Cu") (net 16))
 (segment (start 62.103 107.696) (end 62.103 106.4707) (width 0.25) (layer "F.Cu") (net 16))
 (segment (start 62.8657 106.4707) (end 70.5112 98.8252) (width 0.25) (layer "F.Cu") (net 16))
 (segment (start 108.444 98.8252) (end 122.1722 85.097) (width 0.25) (layer "F.Cu") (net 16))
 (segment (start 70.5112 98.8252) (end 108.444 98.8252) (width 0.25) (layer "F.Cu") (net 16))
 (segment (start 122.1722 85.097) (end 131.064 85.097) (width 0.25) (layer "F.Cu") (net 16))
 (segment (start 62.103 110.236) (end 63.3283 110.236) (width 0.25) (layer "F.Cu") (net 4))
 (segment (start 63.3283 110.236) (end 73.4367 100.1276) (width 0.25) (layer "F.Cu") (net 4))
 (segment (start 109.5494 100.1276) (end 110.864 98.813) (width 0.25) (layer "F.Cu") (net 4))
 (segment (start 73.4367 100.1276) (end 109.5494 100.1276) (width 0.25) (layer "F.Cu") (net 4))
 (segment (start 60.7883 70.363) (end 60.7883 69.9036) (width 0.25) (layer "B.Cu") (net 8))
 (segment (start 59.563 70.363) (end 60.7883 70.363) (width 0.25) (layer "B.Cu") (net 8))
 (segment (start 63.1348 67.5571) (end 70.739 67.5571) (width 0.25) (layer "B.Cu") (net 8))
 (segment (start 70.739 67.5571) (end 70.739 67.557) (width 0.25) (layer "B.Cu") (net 8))
 (segment (start 60.7883 69.9036) (end 63.1348 67.5571) (width 0.25) (layer "B.Cu") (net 8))
 (segment (start 81.4315 84.8655) (end 66.929 70.363) (width 0.25) (layer "B.Cu") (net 17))
 (segment (start 90.4326 84.8655) (end 81.4315 84.8655) (width 0.25) (layer "B.Cu") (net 17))
 (segment (start 90.4326 84.8656) (end 90.4326 84.8655) (width 0.25) (layer "B.Cu") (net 17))
 (segment (start 90.664 85.097) (end 90.4326 84.8656) (width 0.25) (layer "B.Cu") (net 17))
 (segment (start 66.929 70.363) (end 62.103 70.363) (width 0.25) (layer "B.Cu") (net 17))
 (segment (start 97.9968 103.7398) (end 97.014 102.757) (width 0.25) (layer "F.Cu") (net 1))
 (segment (start 133.742 99.575) (end 129.5772 103.7398) (width 0.25) (layer "F.Cu") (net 1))
 (segment (start 129.5772 103.7398) (end 97.9968 103.7398) (width 0.25) (layer "F.Cu") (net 1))
 (segment (start 157.226 99.575) (end 133.742 99.575) (width 0.25) (layer "F.Cu") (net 1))
 (segment (start 80.6726 109.0649) (end 80.1724 108.5647) (width 0.25) (layer "B.Cu") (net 1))
 (segment (start 62.103 92.5353) (end 62.103 80.523) (width 0.25) (layer "B.Cu") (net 1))
 (segment (start 157.226 99.575) (end 157.346 99.695) (width 0.25) (layer "B.Cu") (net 1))
 (segment (start 80.1724 108.5647) (end 78.1324 108.5647) (width 0.25) (layer "B.Cu") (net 1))
 (segment (start 91.0836 107.8465) (end 91.0836 107.9187) (width 0.25) (layer "B.Cu") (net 1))
 (segment (start 89.9374 109.0649) (end 80.6726 109.0649) (width 0.25) (layer "B.Cu") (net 1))
 (segment (start 157.346 99.695) (end 157.346 119.761) (width 0.25) (layer "B.Cu") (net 1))
 (segment (start 91.0836 107.9187) (end 89.9374 109.0649) (width 0.25) (layer "B.Cu") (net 1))
 (segment (start 97.014 102.757) (end 96.1731 102.757) (width 0.25) (layer "B.Cu") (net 1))
 (segment (start 96.1731 102.757) (end 91.0836 107.8465) (width 0.25) (layer "B.Cu") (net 1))
 (segment (start 78.1324 108.5647) (end 62.103 92.5353) (width 0.25) (layer "B.Cu") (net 1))
 (segment (start 90.664 105.297) (end 78.4036 93.0366) (width 0.25) (layer "B.Cu") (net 18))
 (segment (start 60.7883 75.9508) (end 60.7883 75.443) (width 0.25) (layer "B.Cu") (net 18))
 (segment (start 78.4036 93.0366) (end 78.4036 90.7913) (width 0.25) (layer "B.Cu") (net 18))
 (segment (start 61.5505 76.713) (end 60.7883 75.9508) (width 0.25) (layer "B.Cu") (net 18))
 (segment (start 59.563 75.443) (end 60.7883 75.443) (width 0.25) (layer "B.Cu") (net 18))
 (segment (start 64.3253 76.713) (end 61.5505 76.713) (width 0.25) (layer "B.Cu") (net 18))
 (segment (start 78.4036 90.7913) (end 64.3253 76.713) (width 0.25) (layer "B.Cu") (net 18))
 (segment (start 60.7883 72.903) (end 60.7883 72.4435) (width 0.25) (layer "B.Cu") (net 2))
 (segment (start 59.563 72.903) (end 60.7883 72.903) (width 0.25) (layer "B.Cu") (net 2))
 (segment (start 114.0371 95.5743) (end 117.0182 98.5554) (width 0.25) (layer "B.Cu") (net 2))
 (segment (start 90.1697 95.5743) (end 114.0371 95.5743) (width 0.25) (layer "B.Cu") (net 2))
 (segment (start 61.5988 71.633) (end 66.2284 71.633) (width 0.25) (layer "B.Cu") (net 2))
 (segment (start 60.7883 72.4435) (end 61.5988 71.633) (width 0.25) (layer "B.Cu") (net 2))
 (segment (start 66.2284 71.633) (end 90.1697 95.5743) (width 0.25) (layer "B.Cu") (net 2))
 (segment (start 129.0267 98.5554) (end 138.2273 107.756) (width 0.25) (layer "B.Cu") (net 2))
 (segment (start 138.2273 107.756) (end 138.2273 109.5323) (width 0.25) (layer "B.Cu") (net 2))
 (segment (start 138.2273 109.5323) (end 150.996 122.301) (width 0.25) (layer "B.Cu") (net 2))
 (segment (start 117.0182 98.5554) (end 129.0267 98.5554) (width 0.25) (layer "B.Cu") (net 2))
 (segment (start 62.103 72.903) (end 63.3283 72.903) (width 0.25) (layer "F.Cu") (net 12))
 (segment (start 63.3283 72.903) (end 67.5629 77.1376) (width 0.25) (layer "F.Cu") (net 12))
 (segment (start 114.018 77.1376) (end 116.1434 79.263) (width 0.25) (layer "F.Cu") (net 12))
 (segment (start 116.1434 79.263) (end 133.4586 79.263) (width 0.25) (layer "F.Cu") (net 12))
 (segment (start 67.5629 77.1376) (end 114.018 77.1376) (width 0.25) (layer "F.Cu") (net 12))
 (via (at 133.4586 79.263) (size 0.8) (drill 0.4) (layers "F.Cu" "B.Cu") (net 12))
 (segment (start 136.2678 79.263) (end 133.4586 79.263) (width 0.25) (layer "B.Cu") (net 12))
 (segment (start 150.876 102.115) (end 150.876 93.8712) (width 0.25) (layer "B.Cu") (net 12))
 (segment (start 150.876 93.8712) (end 136.2678 79.263) (width 0.25) (layer "B.Cu") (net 12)))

